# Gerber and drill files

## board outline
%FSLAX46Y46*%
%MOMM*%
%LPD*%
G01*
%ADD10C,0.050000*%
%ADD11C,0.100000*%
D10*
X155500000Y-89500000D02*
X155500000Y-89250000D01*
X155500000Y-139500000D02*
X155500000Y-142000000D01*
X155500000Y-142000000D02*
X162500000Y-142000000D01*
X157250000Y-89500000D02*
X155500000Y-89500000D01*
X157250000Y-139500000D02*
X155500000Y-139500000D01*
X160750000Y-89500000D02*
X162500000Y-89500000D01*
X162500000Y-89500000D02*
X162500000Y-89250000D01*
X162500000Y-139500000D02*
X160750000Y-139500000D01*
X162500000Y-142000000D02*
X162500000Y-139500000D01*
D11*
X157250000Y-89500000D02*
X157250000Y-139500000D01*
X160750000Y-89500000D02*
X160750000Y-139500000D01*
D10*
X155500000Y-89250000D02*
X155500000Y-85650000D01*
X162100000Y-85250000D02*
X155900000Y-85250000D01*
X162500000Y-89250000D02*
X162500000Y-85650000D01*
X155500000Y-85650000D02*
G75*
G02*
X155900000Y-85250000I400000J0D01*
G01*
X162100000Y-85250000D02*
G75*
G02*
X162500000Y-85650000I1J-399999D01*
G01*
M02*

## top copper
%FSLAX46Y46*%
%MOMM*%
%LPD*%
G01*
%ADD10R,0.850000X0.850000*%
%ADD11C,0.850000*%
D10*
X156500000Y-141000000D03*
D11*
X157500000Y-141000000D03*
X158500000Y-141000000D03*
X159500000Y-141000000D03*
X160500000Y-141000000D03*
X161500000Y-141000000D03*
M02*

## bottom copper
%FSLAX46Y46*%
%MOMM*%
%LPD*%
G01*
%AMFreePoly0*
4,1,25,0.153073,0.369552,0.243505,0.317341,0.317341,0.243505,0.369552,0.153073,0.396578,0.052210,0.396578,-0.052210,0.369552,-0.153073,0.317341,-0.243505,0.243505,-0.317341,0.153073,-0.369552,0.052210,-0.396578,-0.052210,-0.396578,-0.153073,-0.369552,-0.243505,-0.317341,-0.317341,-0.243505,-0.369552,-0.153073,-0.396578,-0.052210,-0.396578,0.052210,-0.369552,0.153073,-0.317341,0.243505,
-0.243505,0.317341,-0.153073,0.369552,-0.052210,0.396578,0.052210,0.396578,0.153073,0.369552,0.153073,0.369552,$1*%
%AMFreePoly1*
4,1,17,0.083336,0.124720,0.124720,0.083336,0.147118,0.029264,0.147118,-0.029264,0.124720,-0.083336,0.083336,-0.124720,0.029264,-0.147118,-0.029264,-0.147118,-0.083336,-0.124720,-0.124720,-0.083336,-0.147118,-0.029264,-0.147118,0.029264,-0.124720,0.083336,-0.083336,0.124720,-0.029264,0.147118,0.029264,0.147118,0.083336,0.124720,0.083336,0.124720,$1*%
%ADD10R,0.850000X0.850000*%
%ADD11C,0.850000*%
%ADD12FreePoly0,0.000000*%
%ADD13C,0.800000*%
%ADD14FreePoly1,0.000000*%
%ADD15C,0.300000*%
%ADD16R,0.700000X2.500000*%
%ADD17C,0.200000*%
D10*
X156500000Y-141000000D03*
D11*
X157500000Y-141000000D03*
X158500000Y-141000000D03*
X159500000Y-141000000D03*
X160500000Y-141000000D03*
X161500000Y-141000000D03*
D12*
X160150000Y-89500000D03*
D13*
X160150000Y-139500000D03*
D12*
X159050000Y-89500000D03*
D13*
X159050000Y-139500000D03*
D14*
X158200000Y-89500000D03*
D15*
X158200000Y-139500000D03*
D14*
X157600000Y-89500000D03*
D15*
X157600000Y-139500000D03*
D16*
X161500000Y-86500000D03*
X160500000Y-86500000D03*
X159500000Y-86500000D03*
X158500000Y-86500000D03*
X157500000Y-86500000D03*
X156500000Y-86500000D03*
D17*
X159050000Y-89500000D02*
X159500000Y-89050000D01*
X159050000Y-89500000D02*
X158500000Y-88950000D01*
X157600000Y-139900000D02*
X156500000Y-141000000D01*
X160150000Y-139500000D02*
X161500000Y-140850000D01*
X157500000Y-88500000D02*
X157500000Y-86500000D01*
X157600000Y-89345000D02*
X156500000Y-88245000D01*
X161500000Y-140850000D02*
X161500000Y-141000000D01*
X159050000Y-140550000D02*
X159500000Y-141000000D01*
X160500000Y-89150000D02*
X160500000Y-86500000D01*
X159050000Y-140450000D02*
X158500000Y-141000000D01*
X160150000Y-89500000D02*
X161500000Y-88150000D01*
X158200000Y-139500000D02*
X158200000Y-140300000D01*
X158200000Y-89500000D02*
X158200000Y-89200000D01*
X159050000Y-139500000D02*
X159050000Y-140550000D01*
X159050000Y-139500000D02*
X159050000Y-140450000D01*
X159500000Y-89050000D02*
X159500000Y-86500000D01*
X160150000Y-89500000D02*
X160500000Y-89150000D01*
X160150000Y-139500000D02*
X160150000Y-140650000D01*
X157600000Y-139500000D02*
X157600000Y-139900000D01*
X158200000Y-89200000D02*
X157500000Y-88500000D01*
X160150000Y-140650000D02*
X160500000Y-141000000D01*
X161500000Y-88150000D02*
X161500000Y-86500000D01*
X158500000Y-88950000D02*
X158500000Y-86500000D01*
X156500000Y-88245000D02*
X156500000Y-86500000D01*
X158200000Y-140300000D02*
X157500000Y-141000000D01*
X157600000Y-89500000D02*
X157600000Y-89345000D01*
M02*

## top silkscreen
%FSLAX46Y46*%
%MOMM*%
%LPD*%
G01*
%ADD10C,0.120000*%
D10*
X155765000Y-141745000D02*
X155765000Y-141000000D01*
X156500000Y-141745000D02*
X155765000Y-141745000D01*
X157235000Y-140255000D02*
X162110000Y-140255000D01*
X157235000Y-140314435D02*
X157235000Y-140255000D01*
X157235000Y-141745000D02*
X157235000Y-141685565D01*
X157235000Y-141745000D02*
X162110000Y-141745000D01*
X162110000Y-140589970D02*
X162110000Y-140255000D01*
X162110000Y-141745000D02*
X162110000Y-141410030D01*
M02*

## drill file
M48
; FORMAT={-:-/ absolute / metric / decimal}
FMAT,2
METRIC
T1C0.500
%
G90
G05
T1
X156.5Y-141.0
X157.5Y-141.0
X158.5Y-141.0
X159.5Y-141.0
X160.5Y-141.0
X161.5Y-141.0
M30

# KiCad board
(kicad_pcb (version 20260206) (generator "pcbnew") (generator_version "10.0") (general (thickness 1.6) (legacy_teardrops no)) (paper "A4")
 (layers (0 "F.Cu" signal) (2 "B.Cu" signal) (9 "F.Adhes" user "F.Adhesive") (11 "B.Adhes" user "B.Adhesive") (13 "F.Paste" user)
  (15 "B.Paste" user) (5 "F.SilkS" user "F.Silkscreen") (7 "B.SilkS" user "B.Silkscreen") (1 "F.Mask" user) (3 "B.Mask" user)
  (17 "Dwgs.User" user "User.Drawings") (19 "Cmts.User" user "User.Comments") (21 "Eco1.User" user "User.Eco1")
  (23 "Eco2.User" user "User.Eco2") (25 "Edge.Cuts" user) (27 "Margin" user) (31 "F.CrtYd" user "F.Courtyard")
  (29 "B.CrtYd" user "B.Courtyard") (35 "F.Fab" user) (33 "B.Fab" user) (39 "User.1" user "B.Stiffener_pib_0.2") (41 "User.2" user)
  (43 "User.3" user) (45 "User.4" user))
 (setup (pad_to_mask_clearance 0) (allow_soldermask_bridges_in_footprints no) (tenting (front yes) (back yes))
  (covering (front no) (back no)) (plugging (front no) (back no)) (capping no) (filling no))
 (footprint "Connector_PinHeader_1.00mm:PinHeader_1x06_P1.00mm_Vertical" (layer "F.Cu") (at 156.5 141 90)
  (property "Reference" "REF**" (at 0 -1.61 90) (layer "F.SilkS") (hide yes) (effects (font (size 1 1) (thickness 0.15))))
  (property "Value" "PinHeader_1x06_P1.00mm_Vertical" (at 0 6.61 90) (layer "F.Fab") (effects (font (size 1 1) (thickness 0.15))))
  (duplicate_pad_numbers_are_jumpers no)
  (fp_line (start -0.745 -0.735) (end 0 -0.735) (stroke (width 0.12) (type solid)) (layer "F.SilkS"))
  (fp_line (start -0.745 0) (end -0.745 -0.735) (stroke (width 0.12) (type solid)) (layer "F.SilkS"))
  (fp_line (start 0.745 0.735) (end 0.745 5.61) (stroke (width 0.12) (type solid)) (layer "F.SilkS"))
  (fp_line (start 0.685565 0.735) (end 0.745 0.735) (stroke (width 0.12) (type solid)) (layer "F.SilkS"))
  (fp_line (start -0.745 0.735) (end -0.685565 0.735) (stroke (width 0.12) (type solid)) (layer "F.SilkS"))
  (fp_line (start -0.745 0.735) (end -0.745 5.61) (stroke (width 0.12) (type solid)) (layer "F.SilkS"))
  (fp_line (start 0.41003 5.61) (end 0.745 5.61) (stroke (width 0.12) (type solid)) (layer "F.SilkS"))
  (fp_line (start -0.745 5.61) (end -0.41003 5.61) (stroke (width 0.12) (type solid)) (layer "F.SilkS"))
  (pad "1" thru_hole rect (at 0 0 90) (size 0.85 0.85) (drill 0.5) (layers "*.Cu" "*.Mask") (remove_unused_layers no))
  (pad "2" thru_hole circle (at 0 1 90) (size 0.85 0.85) (drill 0.5) (layers "*.Cu" "*.Mask") (remove_unused_layers no))
  (pad "3" thru_hole circle (at 0 2 90) (size 0.85 0.85) (drill 0.5) (layers "*.Cu" "*.Mask") (remove_unused_layers no))
  (pad "4" thru_hole circle (at 0 3 90) (size 0.85 0.85) (drill 0.5) (layers "*.Cu" "*.Mask") (remove_unused_layers no))
  (pad "5" thru_hole circle (at 0 4 90) (size 0.85 0.85) (drill 0.5) (layers "*.Cu" "*.Mask") (remove_unused_layers no))
  (pad "6" thru_hole circle (at 0 5 90) (size 0.85 0.85) (drill 0.5) (layers "*.Cu" "*.Mask") (remove_unused_layers no)))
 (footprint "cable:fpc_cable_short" (layer "F.Cu") (at 159 89.5)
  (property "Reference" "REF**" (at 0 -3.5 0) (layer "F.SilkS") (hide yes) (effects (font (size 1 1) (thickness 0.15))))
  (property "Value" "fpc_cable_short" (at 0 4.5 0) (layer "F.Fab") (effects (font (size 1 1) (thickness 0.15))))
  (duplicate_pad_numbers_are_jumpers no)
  (fp_line (start -1.75 0) (end -1.75 50) (stroke (width 0.1) (type solid)) (layer "Edge.Cuts"))
  (fp_line (start 1.75 0) (end 1.75 50) (stroke (width 0.1) (type solid)) (layer "Edge.Cuts"))
  (pad "1" smd custom (at 1.15 0) (size 0.8 0.8) (layers "B.Cu") (thermal_bridge_angle 90) (options (clearance outline) (anchor circle))
   (primitives))
  (pad "1" smd circle (at 1.15 50) (size 0.8 0.8) (layers "B.Cu"))
  (pad "2" smd custom (at 0.05 0) (size 0.8 0.8) (layers "B.Cu") (thermal_bridge_angle 90) (options (clearance outline) (anchor circle))
   (primitives))
  (pad "2" smd circle (at 0.05 50) (size 0.8 0.8) (layers "B.Cu"))
  (pad "3" smd custom (at -0.8 0) (size 0.3 0.3) (layers "B.Cu") (thermal_bridge_angle 90) (options (clearance outline) (anchor circle))
   (primitives))
  (pad "3" smd circle (at -0.8 50) (size 0.3 0.3) (layers "B.Cu"))
  (pad "4" smd custom (at -1.4 0) (size 0.3 0.3) (layers "B.Cu") (thermal_bridge_angle 90) (options (clearance outline) (anchor circle))
   (primitives))
  (pad "4" smd circle (at -1.4 50) (size 0.3 0.3) (layers "B.Cu")))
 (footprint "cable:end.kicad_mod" (layer "B.Cu") (at 161.5 86.5 180)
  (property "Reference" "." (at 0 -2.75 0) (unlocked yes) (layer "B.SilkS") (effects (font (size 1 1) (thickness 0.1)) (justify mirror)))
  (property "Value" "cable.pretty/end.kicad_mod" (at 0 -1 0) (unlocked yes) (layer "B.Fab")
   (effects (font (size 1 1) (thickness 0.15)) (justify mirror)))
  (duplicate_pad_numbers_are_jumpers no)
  (fp_line (start 6 -2.75) (end 6 0.85) (stroke (width 0.05) (type default)) (layer "Edge.Cuts"))
  (fp_line (start -0.6 1.25) (end 5.6 1.25) (stroke (width 0.05) (type default)) (layer "Edge.Cuts"))
  (fp_line (start -1 -2.75) (end -1 0.85) (stroke (width 0.05) (type default)) (layer "Edge.Cuts"))
  (fp_arc (start 6 0.85) (mid 5.882843 1.132843) (end 5.6 1.25) (stroke (width 0.05) (type default)) (layer "Edge.Cuts"))
  (fp_arc (start -0.6 1.25) (mid -0.882843 1.132843) (end -1 0.85) (stroke (width 0.05) (type default)) (layer "Edge.Cuts"))
  (pad "1" smd rect (at 0 0 90) (size 2.5 0.7) (layers "B.Cu" "B.Mask" "B.Paste"))
  (pad "2" smd rect (at 1 0 90) (size 2.5 0.7) (layers "B.Cu" "B.Mask" "B.Paste"))
  (pad "3" smd rect (at 2 0 90) (size 2.5 0.7) (layers "B.Cu" "B.Mask" "B.Paste"))
  (pad "4" smd rect (at 3 0 90) (size 2.5 0.7) (layers "B.Cu" "B.Mask" "B.Paste"))
  (pad "5" smd rect (at 4 0 90) (size 2.5 0.7) (layers "B.Cu" "B.Mask" "B.Paste"))
  (pad "6" smd rect (at 5 0 90) (size 2.5 0.7) (layers "B.Cu" "B.Mask" "B.Paste")))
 (gr_line (start 155.5 89.5) (end 155.5 89.25) (stroke (width 0.05) (type default)) (layer "Edge.Cuts"))
 (gr_line (start 155.5 139.5) (end 155.5 142) (stroke (width 0.05) (type default)) (layer "Edge.Cuts"))
 (gr_line (start 155.5 142) (end 162.5 142) (stroke (width 0.05) (type default)) (layer "Edge.Cuts"))
 (gr_line (start 157.25 89.5) (end 155.5 89.5) (stroke (width 0.05) (type default)) (layer "Edge.Cuts"))
 (gr_line (start 157.25 139.5) (end 155.5 139.5) (stroke (width 0.05) (type default)) (layer "Edge.Cuts"))
 (gr_line (start 160.75 89.5) (end 162.5 89.5) (stroke (width 0.05) (type default)) (layer "Edge.Cuts"))
 (gr_line (start 162.5 89.5) (end 162.5 89.25) (stroke (width 0.05) (type default)) (layer "Edge.Cuts"))
 (gr_line (start 162.5 139.5) (end 160.75 139.5) (stroke (width 0.05) (type default)) (layer "Edge.Cuts"))
 (gr_line (start 162.5 142) (end 162.5 139.5) (stroke (width 0.05) (type default)) (layer "Edge.Cuts"))
 (segment (start 159.05 89.5) (end 159.5 89.05) (width 0.2) (layer "B.Cu") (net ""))
 (segment (start 159.05 89.5) (end 158.5 88.95) (width 0.2) (layer "B.Cu") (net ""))
 (segment (start 157.6 139.9) (end 156.5 141) (width 0.2) (layer "B.Cu") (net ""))
 (segment (start 160.15 139.5) (end 161.5 140.85) (width 0.2) (layer "B.Cu") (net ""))
 (segment (start 157.5 88.5) (end 157.5 86.5) (width 0.2) (layer "B.Cu") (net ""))
 (segment (start 157.6 89.345) (end 156.5 88.245) (width 0.2) (layer "B.Cu") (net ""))
 (segment (start 161.5 140.85) (end 161.5 141) (width 0.2) (layer "B.Cu") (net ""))
 (segment (start 159.05 140.55) (end 159.5 141) (width 0.2) (layer "B.Cu") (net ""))
 (segment (start 160.5 89.15) (end 160.5 86.5) (width 0.2) (layer "B.Cu") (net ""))
 (segment (start 159.05 140.45) (end 158.5 141) (width 0.2) (layer "B.Cu") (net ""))
 (segment (start 160.15 89.5) (end 161.5 88.15) (width 0.2) (layer "B.Cu") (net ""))
 (segment (start 158.2 139.5) (end 158.2 140.3) (width 0.2) (layer "B.Cu") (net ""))
 (segment (start 158.2 89.5) (end 158.2 89.2) (width 0.2) (layer "B.Cu") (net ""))
 (segment (start 159.05 139.5) (end 159.05 140.55) (width 0.2) (layer "B.Cu") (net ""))
 (segment (start 159.05 139.5) (end 159.05 140.45) (width 0.2) (layer "B.Cu") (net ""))
 (segment (start 159.5 89.05) (end 159.5 86.5) (width 0.2) (layer "B.Cu") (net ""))
 (segment (start 160.15 89.5) (end 160.5 89.15) (width 0.2) (layer "B.Cu") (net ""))
 (segment (start 160.15 139.5) (end 160.15 140.65) (width 0.2) (layer "B.Cu") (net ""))
 (segment (start 157.6 139.5) (end 157.6 139.9) (width 0.2) (layer "B.Cu") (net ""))
 (segment (start 158.2 89.2) (end 157.5 88.5) (width 0.2) (layer "B.Cu") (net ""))
 (segment (start 160.15 140.65) (end 160.5 141) (width 0.2) (layer "B.Cu") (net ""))
 (segment (start 161.5 88.15) (end 161.5 86.5) (width 0.2) (layer "B.Cu") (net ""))
 (segment (start 158.5 88.95) (end 158.5 86.5) (width 0.2) (layer "B.Cu") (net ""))
 (segment (start 156.5 88.245) (end 156.5 86.5) (width 0.2) (layer "B.Cu") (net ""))
 (segment (start 158.2 140.3) (end 157.5 141) (width 0.2) (layer "B.Cu") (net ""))
 (segment (start 157.6 89.5) (end 157.6 89.345) (width 0.2) (layer "B.Cu") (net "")))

